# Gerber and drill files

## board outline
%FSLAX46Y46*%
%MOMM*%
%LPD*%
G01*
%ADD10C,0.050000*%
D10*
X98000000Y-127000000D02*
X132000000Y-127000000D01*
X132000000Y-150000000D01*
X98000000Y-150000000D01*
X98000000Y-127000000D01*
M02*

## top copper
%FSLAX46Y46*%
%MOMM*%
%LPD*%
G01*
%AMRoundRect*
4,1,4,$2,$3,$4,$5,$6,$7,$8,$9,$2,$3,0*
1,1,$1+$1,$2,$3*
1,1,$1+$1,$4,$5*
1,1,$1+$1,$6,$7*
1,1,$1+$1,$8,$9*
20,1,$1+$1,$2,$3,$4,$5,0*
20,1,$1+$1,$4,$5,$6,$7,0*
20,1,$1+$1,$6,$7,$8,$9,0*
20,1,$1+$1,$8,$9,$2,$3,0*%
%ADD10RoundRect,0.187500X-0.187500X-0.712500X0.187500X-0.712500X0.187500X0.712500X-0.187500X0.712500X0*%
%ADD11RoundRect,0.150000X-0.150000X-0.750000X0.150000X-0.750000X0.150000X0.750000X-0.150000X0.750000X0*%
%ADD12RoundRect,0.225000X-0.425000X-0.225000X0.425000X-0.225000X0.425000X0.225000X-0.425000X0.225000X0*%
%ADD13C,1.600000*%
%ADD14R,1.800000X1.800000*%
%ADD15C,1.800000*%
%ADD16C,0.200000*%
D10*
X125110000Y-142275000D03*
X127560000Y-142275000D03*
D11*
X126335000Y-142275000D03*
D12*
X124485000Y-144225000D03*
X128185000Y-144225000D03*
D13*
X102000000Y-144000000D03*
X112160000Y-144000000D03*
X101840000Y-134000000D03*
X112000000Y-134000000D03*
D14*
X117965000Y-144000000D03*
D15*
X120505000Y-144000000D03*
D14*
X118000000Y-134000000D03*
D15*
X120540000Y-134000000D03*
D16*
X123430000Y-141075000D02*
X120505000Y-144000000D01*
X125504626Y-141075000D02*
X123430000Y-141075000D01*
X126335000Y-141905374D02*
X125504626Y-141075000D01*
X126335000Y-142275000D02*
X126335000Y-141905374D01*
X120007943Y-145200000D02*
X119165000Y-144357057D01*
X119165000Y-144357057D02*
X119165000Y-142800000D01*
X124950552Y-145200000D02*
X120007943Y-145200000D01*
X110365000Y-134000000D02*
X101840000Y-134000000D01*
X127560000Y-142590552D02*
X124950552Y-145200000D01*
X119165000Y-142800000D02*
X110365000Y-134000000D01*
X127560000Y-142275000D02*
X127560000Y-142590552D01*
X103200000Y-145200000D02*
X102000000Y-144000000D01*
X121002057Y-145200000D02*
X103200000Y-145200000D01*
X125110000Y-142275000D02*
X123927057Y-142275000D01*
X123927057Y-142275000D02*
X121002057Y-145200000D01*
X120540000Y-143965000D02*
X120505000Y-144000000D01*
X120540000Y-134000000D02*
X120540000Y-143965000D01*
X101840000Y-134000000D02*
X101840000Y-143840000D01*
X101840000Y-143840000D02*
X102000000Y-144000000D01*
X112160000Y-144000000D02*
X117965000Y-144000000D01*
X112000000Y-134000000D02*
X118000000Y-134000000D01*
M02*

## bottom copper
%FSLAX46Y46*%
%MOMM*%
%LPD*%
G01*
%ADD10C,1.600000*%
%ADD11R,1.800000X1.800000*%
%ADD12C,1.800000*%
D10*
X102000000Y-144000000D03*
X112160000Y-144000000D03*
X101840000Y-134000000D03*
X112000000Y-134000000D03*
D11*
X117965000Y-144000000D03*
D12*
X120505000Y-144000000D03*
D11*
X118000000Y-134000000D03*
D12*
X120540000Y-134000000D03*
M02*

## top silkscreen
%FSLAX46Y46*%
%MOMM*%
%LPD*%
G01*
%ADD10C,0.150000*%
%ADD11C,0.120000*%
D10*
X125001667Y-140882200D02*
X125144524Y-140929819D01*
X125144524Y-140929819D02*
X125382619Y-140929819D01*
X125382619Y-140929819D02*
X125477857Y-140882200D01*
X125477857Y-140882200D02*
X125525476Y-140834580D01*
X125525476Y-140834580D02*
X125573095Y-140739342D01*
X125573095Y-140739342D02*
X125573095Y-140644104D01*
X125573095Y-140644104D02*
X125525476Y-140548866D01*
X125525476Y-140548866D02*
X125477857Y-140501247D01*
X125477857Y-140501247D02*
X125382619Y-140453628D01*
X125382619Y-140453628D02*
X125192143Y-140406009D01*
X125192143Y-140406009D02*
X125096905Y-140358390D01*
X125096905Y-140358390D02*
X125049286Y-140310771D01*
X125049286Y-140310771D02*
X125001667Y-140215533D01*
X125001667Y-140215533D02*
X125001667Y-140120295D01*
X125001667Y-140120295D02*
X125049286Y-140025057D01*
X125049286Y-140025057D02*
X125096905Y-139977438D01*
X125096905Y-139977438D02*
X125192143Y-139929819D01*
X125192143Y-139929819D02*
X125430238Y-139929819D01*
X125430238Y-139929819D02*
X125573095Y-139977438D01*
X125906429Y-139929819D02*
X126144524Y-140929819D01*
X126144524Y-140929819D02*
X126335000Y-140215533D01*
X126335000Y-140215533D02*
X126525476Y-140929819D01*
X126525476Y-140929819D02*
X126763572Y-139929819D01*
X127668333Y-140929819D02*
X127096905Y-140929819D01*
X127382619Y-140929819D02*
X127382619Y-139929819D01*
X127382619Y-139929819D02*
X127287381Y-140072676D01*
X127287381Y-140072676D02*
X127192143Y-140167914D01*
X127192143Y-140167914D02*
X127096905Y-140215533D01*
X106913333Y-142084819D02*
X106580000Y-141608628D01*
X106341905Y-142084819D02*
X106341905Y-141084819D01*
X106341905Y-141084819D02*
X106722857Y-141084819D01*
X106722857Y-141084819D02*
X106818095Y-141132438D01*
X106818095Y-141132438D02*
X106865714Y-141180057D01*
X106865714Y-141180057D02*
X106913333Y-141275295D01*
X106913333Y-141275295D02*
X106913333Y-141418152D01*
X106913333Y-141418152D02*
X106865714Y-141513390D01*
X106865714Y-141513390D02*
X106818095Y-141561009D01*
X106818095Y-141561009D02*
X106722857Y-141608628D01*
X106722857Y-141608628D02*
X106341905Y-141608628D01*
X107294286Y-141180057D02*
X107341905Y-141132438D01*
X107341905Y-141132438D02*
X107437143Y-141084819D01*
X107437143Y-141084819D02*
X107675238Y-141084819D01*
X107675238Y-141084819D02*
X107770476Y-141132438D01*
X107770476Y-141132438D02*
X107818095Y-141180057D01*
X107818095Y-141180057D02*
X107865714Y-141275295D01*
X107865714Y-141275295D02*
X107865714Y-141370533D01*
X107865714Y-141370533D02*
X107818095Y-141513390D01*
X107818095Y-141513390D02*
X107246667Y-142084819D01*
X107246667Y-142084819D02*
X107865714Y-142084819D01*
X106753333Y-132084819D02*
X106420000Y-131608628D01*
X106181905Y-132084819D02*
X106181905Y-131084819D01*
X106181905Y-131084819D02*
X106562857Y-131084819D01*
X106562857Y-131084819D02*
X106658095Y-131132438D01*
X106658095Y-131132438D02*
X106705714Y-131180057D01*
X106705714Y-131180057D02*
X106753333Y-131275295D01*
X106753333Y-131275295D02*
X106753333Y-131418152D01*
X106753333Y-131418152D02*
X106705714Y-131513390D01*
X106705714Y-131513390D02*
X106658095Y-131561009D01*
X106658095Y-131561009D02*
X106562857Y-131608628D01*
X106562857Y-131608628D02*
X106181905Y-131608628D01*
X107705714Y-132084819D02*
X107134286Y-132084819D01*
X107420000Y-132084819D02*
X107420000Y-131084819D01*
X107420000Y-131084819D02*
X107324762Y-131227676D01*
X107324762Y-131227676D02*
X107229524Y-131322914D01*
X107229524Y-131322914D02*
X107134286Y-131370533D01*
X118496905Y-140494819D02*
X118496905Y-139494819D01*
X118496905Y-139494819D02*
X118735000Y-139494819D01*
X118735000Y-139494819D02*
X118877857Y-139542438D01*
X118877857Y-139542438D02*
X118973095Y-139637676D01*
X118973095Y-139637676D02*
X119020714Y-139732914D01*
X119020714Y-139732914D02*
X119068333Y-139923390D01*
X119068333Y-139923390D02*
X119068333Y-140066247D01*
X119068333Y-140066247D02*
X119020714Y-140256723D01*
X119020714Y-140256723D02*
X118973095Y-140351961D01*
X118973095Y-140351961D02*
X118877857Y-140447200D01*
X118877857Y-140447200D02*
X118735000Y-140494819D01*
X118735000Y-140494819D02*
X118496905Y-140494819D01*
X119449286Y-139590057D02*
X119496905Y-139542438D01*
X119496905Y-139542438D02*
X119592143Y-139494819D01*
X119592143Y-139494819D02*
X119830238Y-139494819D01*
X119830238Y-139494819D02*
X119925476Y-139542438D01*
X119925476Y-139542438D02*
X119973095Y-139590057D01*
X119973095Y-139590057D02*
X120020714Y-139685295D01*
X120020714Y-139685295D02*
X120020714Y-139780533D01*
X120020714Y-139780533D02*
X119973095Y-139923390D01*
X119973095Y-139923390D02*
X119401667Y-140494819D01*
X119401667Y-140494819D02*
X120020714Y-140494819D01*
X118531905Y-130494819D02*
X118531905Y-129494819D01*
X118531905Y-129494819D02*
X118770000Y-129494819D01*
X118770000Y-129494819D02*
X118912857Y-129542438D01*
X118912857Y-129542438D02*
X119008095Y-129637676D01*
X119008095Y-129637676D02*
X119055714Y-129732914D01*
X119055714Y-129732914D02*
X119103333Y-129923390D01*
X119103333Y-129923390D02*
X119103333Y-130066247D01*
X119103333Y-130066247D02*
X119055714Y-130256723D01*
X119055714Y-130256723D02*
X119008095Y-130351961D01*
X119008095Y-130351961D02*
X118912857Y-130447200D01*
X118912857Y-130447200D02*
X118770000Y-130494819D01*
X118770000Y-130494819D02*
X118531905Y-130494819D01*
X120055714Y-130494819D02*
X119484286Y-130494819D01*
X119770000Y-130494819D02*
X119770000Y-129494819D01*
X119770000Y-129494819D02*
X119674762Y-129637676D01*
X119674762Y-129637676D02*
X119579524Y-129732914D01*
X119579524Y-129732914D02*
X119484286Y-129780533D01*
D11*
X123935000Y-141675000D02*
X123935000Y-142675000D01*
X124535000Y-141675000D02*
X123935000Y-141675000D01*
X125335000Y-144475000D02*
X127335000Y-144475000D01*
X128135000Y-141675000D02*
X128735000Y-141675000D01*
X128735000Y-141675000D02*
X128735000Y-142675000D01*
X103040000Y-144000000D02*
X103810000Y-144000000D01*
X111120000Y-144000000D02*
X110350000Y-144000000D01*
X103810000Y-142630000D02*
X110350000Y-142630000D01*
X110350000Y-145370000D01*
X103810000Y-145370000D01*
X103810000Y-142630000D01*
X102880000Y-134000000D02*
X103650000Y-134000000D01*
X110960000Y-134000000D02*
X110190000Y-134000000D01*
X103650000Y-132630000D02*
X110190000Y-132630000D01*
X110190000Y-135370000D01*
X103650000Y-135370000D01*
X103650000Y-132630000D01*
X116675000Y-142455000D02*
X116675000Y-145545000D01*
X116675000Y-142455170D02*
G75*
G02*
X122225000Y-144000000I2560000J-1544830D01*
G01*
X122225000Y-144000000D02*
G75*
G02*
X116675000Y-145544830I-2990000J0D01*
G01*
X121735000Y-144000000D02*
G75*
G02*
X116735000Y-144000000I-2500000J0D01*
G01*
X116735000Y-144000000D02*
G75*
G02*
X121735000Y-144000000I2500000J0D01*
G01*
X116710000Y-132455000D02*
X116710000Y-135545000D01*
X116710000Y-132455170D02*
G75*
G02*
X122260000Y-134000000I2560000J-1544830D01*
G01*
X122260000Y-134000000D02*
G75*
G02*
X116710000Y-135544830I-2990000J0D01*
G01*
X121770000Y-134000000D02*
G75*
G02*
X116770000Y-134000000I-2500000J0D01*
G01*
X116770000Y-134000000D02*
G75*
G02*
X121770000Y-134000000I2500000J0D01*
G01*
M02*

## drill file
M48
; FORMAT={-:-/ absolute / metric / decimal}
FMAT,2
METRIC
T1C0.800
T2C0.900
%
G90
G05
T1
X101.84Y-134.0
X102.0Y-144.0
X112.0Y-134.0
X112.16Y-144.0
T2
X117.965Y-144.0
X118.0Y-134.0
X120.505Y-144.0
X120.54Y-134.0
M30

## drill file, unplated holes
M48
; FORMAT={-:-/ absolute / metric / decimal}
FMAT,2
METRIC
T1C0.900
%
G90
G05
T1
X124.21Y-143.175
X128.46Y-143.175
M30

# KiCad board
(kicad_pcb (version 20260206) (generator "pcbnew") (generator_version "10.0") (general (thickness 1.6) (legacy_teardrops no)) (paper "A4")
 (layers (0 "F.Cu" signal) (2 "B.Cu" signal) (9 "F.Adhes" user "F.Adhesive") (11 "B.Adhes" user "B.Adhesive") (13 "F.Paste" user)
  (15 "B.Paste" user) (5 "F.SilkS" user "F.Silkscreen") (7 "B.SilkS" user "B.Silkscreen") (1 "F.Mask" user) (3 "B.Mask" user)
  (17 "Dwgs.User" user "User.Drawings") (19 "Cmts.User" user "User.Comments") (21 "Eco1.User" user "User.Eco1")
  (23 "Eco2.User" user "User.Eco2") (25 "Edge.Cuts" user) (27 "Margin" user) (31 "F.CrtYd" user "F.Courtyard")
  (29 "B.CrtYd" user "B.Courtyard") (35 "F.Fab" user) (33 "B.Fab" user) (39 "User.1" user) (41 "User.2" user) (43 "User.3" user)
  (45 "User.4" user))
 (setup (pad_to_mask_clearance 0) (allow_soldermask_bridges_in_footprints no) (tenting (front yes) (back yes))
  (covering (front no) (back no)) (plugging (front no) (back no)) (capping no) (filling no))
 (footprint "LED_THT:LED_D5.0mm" (layer "F.Cu") (at 118 134)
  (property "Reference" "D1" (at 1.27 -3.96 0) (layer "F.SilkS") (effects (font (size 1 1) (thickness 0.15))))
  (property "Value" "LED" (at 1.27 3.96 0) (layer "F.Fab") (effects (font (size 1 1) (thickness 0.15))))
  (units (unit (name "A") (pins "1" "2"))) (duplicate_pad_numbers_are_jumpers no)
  (fp_line (start -1.29 -1.545) (end -1.29 1.545) (stroke (width 0.12) (type solid)) (layer "F.SilkS"))
  (fp_arc (start -1.29 -1.54483) (mid 2.071779 -2.880495) (end 4.26 0) (stroke (width 0.12) (type solid)) (layer "F.SilkS"))
  (fp_arc (start 4.26 0) (mid 2.071779 2.880495) (end -1.29 1.54483) (stroke (width 0.12) (type solid)) (layer "F.SilkS"))
  (fp_circle (center 1.27 0) (end 3.77 0) (stroke (width 0.12) (type solid)) (fill no) (layer "F.SilkS"))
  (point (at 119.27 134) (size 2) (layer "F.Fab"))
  (pad "1" thru_hole rect (at 0 0) (size 1.8 1.8) (drill 0.9) (layers "*.Cu" "*.Mask") (remove_unused_layers no) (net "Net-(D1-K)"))
  (pad "2" thru_hole circle (at 2.54 0) (size 1.8 1.8) (drill 0.9) (layers "*.Cu" "*.Mask") (remove_unused_layers no) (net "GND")))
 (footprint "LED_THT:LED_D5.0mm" (layer "F.Cu") (at 117.965 144)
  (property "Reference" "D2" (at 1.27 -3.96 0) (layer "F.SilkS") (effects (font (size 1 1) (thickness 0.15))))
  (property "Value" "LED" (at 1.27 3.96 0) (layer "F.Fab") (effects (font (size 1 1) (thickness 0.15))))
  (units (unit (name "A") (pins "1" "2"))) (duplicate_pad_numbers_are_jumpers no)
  (fp_line (start -1.29 -1.545) (end -1.29 1.545) (stroke (width 0.12) (type solid)) (layer "F.SilkS"))
  (fp_arc (start -1.29 -1.54483) (mid 2.071779 -2.880495) (end 4.26 0) (stroke (width 0.12) (type solid)) (layer "F.SilkS"))
  (fp_arc (start 4.26 0) (mid 2.071779 2.880495) (end -1.29 1.54483) (stroke (width 0.12) (type solid)) (layer "F.SilkS"))
  (fp_circle (center 1.27 0) (end 3.77 0) (stroke (width 0.12) (type solid)) (fill no) (layer "F.SilkS"))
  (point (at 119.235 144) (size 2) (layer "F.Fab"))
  (pad "1" thru_hole rect (at 0 0) (size 1.8 1.8) (drill 0.9) (layers "*.Cu" "*.Mask") (remove_unused_layers no) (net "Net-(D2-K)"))
  (pad "2" thru_hole circle (at 2.54 0) (size 1.8 1.8) (drill 0.9) (layers "*.Cu" "*.Mask") (remove_unused_layers no) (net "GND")))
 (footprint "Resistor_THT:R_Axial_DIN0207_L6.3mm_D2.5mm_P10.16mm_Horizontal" (layer "F.Cu") (at 102 144)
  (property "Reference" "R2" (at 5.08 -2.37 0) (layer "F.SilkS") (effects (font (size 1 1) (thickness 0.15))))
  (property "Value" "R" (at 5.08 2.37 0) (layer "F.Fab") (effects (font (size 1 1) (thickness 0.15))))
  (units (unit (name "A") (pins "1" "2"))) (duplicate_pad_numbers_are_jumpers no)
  (fp_line (start 1.04 0) (end 1.81 0) (stroke (width 0.12) (type solid)) (layer "F.SilkS"))
  (fp_line (start 9.12 0) (end 8.35 0) (stroke (width 0.12) (type solid)) (layer "F.SilkS"))
  (fp_rect (start 1.81 -1.37) (end 8.35 1.37) (stroke (width 0.12) (type solid)) (fill no) (layer "F.SilkS"))
  (pad "1" thru_hole circle (at 0 0) (size 1.6 1.6) (drill 0.8) (layers "*.Cu" "*.Mask") (remove_unused_layers no) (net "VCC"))
  (pad "2" thru_hole circle (at 10.16 0) (size 1.6 1.6) (drill 0.8) (layers "*.Cu" "*.Mask") (remove_unused_layers no) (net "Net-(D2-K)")))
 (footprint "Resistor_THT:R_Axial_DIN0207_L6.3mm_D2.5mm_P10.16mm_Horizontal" (layer "F.Cu") (at 101.84 134)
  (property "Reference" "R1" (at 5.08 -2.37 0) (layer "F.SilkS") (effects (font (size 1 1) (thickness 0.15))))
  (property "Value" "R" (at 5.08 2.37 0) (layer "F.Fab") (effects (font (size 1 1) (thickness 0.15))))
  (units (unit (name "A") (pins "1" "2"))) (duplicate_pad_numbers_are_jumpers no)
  (fp_line (start 1.04 0) (end 1.81 0) (stroke (width 0.12) (type solid)) (layer "F.SilkS"))
  (fp_line (start 9.12 0) (end 8.35 0) (stroke (width 0.12) (type solid)) (layer "F.SilkS"))
  (fp_rect (start 1.81 -1.37) (end 8.35 1.37) (stroke (width 0.12) (type solid)) (fill no) (layer "F.SilkS"))
  (pad "1" thru_hole circle (at 0 0) (size 1.6 1.6) (drill 0.8) (layers "*.Cu" "*.Mask") (remove_unused_layers no) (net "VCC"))
  (pad "2" thru_hole circle (at 10.16 0) (size 1.6 1.6) (drill 0.8) (layers "*.Cu" "*.Mask") (remove_unused_layers no) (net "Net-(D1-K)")))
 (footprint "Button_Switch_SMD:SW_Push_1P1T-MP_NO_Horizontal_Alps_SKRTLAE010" (layer "F.Cu") (at 126.335 143.175)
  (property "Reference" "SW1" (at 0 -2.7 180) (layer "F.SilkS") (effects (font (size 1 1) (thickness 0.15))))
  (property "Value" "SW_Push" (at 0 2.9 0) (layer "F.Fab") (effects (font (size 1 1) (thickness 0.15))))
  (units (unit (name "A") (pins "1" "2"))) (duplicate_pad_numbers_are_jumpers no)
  (fp_line (start -2.4 -1.5) (end -2.4 -0.5) (stroke (width 0.12) (type solid)) (layer "F.SilkS"))
  (fp_line (start -1.8 -1.5) (end -2.4 -1.5) (stroke (width 0.12) (type solid)) (layer "F.SilkS"))
  (fp_line (start -1 1.3) (end 1 1.3) (stroke (width 0.12) (type solid)) (layer "F.SilkS"))
  (fp_line (start 1.8 -1.5) (end 2.4 -1.5) (stroke (width 0.12) (type solid)) (layer "F.SilkS"))
  (fp_line (start 2.4 -1.5) (end 2.4 -0.5) (stroke (width 0.12) (type solid)) (layer "F.SilkS"))
  (pad "" np_thru_hole circle (at -2.125 0) (size 0.9 0.9) (drill 0.9) (layers "*.Cu" "*.Mask"))
  (pad "" np_thru_hole circle (at 2.125 0) (size 0.9 0.9) (drill 0.9) (layers "*.Cu" "*.Mask"))
  (pad "1" smd roundrect (at -1.225 -0.9) (size 0.75 1.8) (layers "F.Cu" "F.Mask" "F.Paste") (roundrect_rratio 0.25) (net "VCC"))
  (pad "1" smd roundrect (at 1.225 -0.9) (size 0.75 1.8) (layers "F.Cu" "F.Mask" "F.Paste") (roundrect_rratio 0.25) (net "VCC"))
  (pad "2" smd roundrect (at 0 -0.9) (size 0.6 1.8) (layers "F.Cu" "F.Mask" "F.Paste") (roundrect_rratio 0.25) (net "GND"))
  (pad "MP" smd roundrect (at -1.85 1.05) (size 1.3 0.9) (layers "F.Cu" "F.Mask" "F.Paste") (roundrect_rratio 0.25))
  (pad "MP" smd roundrect (at 1.85 1.05) (size 1.3 0.9) (layers "F.Cu" "F.Mask" "F.Paste") (roundrect_rratio 0.25)))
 (gr_rect (start 98 127) (end 132 150) (stroke (width 0.05) (type default)) (fill no) (layer "Edge.Cuts"))
 (segment (start 123.43 141.075) (end 120.505 144) (width 0.2) (layer "F.Cu") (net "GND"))
 (segment (start 120.54 134) (end 120.54 143.965) (width 0.2) (layer "F.Cu") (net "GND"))
 (segment (start 125.504626 141.075) (end 123.43 141.075) (width 0.2) (layer "F.Cu") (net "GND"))
 (segment (start 120.54 143.965) (end 120.505 144) (width 0.2) (layer "F.Cu") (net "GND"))
 (segment (start 126.335 142.275) (end 126.335 141.905374) (width 0.2) (layer "F.Cu") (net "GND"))
 (segment (start 126.335 141.905374) (end 125.504626 141.075) (width 0.2) (layer "F.Cu") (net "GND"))
 (segment (start 123.927057 142.275) (end 121.002057 145.2) (width 0.2) (layer "F.Cu") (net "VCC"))
 (segment (start 103.2 145.2) (end 102 144) (width 0.2) (layer "F.Cu") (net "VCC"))
 (segment (start 101.84 134) (end 101.84 143.84) (width 0.2) (layer "F.Cu") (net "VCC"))
 (segment (start 119.165 144.357057) (end 119.165 142.8) (width 0.2) (layer "F.Cu") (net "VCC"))
 (segment (start 127.56 142.590552) (end 124.950552 145.2) (width 0.2) (layer "F.Cu") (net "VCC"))
 (segment (start 120.007943 145.2) (end 119.165 144.357057) (width 0.2) (layer "F.Cu") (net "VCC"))
 (segment (start 101.84 143.84) (end 102 144) (width 0.2) (layer "F.Cu") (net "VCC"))
 (segment (start 125.11 142.275) (end 123.927057 142.275) (width 0.2) (layer "F.Cu") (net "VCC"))
 (segment (start 110.365 134) (end 101.84 134) (width 0.2) (layer "F.Cu") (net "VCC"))
 (segment (start 127.56 142.275) (end 127.56 142.590552) (width 0.2) (layer "F.Cu") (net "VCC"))
 (segment (start 121.002057 145.2) (end 103.2 145.2) (width 0.2) (layer "F.Cu") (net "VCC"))
 (segment (start 124.950552 145.2) (end 120.007943 145.2) (width 0.2) (layer "F.Cu") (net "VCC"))
 (segment (start 119.165 142.8) (end 110.365 134) (width 0.2) (layer "F.Cu") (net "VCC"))
 (segment (start 112 134) (end 118 134) (width 0.2) (layer "F.Cu") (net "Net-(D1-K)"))
 (segment (start 112.16 144) (end 117.965 144) (width 0.2) (layer "F.Cu") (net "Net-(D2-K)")))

